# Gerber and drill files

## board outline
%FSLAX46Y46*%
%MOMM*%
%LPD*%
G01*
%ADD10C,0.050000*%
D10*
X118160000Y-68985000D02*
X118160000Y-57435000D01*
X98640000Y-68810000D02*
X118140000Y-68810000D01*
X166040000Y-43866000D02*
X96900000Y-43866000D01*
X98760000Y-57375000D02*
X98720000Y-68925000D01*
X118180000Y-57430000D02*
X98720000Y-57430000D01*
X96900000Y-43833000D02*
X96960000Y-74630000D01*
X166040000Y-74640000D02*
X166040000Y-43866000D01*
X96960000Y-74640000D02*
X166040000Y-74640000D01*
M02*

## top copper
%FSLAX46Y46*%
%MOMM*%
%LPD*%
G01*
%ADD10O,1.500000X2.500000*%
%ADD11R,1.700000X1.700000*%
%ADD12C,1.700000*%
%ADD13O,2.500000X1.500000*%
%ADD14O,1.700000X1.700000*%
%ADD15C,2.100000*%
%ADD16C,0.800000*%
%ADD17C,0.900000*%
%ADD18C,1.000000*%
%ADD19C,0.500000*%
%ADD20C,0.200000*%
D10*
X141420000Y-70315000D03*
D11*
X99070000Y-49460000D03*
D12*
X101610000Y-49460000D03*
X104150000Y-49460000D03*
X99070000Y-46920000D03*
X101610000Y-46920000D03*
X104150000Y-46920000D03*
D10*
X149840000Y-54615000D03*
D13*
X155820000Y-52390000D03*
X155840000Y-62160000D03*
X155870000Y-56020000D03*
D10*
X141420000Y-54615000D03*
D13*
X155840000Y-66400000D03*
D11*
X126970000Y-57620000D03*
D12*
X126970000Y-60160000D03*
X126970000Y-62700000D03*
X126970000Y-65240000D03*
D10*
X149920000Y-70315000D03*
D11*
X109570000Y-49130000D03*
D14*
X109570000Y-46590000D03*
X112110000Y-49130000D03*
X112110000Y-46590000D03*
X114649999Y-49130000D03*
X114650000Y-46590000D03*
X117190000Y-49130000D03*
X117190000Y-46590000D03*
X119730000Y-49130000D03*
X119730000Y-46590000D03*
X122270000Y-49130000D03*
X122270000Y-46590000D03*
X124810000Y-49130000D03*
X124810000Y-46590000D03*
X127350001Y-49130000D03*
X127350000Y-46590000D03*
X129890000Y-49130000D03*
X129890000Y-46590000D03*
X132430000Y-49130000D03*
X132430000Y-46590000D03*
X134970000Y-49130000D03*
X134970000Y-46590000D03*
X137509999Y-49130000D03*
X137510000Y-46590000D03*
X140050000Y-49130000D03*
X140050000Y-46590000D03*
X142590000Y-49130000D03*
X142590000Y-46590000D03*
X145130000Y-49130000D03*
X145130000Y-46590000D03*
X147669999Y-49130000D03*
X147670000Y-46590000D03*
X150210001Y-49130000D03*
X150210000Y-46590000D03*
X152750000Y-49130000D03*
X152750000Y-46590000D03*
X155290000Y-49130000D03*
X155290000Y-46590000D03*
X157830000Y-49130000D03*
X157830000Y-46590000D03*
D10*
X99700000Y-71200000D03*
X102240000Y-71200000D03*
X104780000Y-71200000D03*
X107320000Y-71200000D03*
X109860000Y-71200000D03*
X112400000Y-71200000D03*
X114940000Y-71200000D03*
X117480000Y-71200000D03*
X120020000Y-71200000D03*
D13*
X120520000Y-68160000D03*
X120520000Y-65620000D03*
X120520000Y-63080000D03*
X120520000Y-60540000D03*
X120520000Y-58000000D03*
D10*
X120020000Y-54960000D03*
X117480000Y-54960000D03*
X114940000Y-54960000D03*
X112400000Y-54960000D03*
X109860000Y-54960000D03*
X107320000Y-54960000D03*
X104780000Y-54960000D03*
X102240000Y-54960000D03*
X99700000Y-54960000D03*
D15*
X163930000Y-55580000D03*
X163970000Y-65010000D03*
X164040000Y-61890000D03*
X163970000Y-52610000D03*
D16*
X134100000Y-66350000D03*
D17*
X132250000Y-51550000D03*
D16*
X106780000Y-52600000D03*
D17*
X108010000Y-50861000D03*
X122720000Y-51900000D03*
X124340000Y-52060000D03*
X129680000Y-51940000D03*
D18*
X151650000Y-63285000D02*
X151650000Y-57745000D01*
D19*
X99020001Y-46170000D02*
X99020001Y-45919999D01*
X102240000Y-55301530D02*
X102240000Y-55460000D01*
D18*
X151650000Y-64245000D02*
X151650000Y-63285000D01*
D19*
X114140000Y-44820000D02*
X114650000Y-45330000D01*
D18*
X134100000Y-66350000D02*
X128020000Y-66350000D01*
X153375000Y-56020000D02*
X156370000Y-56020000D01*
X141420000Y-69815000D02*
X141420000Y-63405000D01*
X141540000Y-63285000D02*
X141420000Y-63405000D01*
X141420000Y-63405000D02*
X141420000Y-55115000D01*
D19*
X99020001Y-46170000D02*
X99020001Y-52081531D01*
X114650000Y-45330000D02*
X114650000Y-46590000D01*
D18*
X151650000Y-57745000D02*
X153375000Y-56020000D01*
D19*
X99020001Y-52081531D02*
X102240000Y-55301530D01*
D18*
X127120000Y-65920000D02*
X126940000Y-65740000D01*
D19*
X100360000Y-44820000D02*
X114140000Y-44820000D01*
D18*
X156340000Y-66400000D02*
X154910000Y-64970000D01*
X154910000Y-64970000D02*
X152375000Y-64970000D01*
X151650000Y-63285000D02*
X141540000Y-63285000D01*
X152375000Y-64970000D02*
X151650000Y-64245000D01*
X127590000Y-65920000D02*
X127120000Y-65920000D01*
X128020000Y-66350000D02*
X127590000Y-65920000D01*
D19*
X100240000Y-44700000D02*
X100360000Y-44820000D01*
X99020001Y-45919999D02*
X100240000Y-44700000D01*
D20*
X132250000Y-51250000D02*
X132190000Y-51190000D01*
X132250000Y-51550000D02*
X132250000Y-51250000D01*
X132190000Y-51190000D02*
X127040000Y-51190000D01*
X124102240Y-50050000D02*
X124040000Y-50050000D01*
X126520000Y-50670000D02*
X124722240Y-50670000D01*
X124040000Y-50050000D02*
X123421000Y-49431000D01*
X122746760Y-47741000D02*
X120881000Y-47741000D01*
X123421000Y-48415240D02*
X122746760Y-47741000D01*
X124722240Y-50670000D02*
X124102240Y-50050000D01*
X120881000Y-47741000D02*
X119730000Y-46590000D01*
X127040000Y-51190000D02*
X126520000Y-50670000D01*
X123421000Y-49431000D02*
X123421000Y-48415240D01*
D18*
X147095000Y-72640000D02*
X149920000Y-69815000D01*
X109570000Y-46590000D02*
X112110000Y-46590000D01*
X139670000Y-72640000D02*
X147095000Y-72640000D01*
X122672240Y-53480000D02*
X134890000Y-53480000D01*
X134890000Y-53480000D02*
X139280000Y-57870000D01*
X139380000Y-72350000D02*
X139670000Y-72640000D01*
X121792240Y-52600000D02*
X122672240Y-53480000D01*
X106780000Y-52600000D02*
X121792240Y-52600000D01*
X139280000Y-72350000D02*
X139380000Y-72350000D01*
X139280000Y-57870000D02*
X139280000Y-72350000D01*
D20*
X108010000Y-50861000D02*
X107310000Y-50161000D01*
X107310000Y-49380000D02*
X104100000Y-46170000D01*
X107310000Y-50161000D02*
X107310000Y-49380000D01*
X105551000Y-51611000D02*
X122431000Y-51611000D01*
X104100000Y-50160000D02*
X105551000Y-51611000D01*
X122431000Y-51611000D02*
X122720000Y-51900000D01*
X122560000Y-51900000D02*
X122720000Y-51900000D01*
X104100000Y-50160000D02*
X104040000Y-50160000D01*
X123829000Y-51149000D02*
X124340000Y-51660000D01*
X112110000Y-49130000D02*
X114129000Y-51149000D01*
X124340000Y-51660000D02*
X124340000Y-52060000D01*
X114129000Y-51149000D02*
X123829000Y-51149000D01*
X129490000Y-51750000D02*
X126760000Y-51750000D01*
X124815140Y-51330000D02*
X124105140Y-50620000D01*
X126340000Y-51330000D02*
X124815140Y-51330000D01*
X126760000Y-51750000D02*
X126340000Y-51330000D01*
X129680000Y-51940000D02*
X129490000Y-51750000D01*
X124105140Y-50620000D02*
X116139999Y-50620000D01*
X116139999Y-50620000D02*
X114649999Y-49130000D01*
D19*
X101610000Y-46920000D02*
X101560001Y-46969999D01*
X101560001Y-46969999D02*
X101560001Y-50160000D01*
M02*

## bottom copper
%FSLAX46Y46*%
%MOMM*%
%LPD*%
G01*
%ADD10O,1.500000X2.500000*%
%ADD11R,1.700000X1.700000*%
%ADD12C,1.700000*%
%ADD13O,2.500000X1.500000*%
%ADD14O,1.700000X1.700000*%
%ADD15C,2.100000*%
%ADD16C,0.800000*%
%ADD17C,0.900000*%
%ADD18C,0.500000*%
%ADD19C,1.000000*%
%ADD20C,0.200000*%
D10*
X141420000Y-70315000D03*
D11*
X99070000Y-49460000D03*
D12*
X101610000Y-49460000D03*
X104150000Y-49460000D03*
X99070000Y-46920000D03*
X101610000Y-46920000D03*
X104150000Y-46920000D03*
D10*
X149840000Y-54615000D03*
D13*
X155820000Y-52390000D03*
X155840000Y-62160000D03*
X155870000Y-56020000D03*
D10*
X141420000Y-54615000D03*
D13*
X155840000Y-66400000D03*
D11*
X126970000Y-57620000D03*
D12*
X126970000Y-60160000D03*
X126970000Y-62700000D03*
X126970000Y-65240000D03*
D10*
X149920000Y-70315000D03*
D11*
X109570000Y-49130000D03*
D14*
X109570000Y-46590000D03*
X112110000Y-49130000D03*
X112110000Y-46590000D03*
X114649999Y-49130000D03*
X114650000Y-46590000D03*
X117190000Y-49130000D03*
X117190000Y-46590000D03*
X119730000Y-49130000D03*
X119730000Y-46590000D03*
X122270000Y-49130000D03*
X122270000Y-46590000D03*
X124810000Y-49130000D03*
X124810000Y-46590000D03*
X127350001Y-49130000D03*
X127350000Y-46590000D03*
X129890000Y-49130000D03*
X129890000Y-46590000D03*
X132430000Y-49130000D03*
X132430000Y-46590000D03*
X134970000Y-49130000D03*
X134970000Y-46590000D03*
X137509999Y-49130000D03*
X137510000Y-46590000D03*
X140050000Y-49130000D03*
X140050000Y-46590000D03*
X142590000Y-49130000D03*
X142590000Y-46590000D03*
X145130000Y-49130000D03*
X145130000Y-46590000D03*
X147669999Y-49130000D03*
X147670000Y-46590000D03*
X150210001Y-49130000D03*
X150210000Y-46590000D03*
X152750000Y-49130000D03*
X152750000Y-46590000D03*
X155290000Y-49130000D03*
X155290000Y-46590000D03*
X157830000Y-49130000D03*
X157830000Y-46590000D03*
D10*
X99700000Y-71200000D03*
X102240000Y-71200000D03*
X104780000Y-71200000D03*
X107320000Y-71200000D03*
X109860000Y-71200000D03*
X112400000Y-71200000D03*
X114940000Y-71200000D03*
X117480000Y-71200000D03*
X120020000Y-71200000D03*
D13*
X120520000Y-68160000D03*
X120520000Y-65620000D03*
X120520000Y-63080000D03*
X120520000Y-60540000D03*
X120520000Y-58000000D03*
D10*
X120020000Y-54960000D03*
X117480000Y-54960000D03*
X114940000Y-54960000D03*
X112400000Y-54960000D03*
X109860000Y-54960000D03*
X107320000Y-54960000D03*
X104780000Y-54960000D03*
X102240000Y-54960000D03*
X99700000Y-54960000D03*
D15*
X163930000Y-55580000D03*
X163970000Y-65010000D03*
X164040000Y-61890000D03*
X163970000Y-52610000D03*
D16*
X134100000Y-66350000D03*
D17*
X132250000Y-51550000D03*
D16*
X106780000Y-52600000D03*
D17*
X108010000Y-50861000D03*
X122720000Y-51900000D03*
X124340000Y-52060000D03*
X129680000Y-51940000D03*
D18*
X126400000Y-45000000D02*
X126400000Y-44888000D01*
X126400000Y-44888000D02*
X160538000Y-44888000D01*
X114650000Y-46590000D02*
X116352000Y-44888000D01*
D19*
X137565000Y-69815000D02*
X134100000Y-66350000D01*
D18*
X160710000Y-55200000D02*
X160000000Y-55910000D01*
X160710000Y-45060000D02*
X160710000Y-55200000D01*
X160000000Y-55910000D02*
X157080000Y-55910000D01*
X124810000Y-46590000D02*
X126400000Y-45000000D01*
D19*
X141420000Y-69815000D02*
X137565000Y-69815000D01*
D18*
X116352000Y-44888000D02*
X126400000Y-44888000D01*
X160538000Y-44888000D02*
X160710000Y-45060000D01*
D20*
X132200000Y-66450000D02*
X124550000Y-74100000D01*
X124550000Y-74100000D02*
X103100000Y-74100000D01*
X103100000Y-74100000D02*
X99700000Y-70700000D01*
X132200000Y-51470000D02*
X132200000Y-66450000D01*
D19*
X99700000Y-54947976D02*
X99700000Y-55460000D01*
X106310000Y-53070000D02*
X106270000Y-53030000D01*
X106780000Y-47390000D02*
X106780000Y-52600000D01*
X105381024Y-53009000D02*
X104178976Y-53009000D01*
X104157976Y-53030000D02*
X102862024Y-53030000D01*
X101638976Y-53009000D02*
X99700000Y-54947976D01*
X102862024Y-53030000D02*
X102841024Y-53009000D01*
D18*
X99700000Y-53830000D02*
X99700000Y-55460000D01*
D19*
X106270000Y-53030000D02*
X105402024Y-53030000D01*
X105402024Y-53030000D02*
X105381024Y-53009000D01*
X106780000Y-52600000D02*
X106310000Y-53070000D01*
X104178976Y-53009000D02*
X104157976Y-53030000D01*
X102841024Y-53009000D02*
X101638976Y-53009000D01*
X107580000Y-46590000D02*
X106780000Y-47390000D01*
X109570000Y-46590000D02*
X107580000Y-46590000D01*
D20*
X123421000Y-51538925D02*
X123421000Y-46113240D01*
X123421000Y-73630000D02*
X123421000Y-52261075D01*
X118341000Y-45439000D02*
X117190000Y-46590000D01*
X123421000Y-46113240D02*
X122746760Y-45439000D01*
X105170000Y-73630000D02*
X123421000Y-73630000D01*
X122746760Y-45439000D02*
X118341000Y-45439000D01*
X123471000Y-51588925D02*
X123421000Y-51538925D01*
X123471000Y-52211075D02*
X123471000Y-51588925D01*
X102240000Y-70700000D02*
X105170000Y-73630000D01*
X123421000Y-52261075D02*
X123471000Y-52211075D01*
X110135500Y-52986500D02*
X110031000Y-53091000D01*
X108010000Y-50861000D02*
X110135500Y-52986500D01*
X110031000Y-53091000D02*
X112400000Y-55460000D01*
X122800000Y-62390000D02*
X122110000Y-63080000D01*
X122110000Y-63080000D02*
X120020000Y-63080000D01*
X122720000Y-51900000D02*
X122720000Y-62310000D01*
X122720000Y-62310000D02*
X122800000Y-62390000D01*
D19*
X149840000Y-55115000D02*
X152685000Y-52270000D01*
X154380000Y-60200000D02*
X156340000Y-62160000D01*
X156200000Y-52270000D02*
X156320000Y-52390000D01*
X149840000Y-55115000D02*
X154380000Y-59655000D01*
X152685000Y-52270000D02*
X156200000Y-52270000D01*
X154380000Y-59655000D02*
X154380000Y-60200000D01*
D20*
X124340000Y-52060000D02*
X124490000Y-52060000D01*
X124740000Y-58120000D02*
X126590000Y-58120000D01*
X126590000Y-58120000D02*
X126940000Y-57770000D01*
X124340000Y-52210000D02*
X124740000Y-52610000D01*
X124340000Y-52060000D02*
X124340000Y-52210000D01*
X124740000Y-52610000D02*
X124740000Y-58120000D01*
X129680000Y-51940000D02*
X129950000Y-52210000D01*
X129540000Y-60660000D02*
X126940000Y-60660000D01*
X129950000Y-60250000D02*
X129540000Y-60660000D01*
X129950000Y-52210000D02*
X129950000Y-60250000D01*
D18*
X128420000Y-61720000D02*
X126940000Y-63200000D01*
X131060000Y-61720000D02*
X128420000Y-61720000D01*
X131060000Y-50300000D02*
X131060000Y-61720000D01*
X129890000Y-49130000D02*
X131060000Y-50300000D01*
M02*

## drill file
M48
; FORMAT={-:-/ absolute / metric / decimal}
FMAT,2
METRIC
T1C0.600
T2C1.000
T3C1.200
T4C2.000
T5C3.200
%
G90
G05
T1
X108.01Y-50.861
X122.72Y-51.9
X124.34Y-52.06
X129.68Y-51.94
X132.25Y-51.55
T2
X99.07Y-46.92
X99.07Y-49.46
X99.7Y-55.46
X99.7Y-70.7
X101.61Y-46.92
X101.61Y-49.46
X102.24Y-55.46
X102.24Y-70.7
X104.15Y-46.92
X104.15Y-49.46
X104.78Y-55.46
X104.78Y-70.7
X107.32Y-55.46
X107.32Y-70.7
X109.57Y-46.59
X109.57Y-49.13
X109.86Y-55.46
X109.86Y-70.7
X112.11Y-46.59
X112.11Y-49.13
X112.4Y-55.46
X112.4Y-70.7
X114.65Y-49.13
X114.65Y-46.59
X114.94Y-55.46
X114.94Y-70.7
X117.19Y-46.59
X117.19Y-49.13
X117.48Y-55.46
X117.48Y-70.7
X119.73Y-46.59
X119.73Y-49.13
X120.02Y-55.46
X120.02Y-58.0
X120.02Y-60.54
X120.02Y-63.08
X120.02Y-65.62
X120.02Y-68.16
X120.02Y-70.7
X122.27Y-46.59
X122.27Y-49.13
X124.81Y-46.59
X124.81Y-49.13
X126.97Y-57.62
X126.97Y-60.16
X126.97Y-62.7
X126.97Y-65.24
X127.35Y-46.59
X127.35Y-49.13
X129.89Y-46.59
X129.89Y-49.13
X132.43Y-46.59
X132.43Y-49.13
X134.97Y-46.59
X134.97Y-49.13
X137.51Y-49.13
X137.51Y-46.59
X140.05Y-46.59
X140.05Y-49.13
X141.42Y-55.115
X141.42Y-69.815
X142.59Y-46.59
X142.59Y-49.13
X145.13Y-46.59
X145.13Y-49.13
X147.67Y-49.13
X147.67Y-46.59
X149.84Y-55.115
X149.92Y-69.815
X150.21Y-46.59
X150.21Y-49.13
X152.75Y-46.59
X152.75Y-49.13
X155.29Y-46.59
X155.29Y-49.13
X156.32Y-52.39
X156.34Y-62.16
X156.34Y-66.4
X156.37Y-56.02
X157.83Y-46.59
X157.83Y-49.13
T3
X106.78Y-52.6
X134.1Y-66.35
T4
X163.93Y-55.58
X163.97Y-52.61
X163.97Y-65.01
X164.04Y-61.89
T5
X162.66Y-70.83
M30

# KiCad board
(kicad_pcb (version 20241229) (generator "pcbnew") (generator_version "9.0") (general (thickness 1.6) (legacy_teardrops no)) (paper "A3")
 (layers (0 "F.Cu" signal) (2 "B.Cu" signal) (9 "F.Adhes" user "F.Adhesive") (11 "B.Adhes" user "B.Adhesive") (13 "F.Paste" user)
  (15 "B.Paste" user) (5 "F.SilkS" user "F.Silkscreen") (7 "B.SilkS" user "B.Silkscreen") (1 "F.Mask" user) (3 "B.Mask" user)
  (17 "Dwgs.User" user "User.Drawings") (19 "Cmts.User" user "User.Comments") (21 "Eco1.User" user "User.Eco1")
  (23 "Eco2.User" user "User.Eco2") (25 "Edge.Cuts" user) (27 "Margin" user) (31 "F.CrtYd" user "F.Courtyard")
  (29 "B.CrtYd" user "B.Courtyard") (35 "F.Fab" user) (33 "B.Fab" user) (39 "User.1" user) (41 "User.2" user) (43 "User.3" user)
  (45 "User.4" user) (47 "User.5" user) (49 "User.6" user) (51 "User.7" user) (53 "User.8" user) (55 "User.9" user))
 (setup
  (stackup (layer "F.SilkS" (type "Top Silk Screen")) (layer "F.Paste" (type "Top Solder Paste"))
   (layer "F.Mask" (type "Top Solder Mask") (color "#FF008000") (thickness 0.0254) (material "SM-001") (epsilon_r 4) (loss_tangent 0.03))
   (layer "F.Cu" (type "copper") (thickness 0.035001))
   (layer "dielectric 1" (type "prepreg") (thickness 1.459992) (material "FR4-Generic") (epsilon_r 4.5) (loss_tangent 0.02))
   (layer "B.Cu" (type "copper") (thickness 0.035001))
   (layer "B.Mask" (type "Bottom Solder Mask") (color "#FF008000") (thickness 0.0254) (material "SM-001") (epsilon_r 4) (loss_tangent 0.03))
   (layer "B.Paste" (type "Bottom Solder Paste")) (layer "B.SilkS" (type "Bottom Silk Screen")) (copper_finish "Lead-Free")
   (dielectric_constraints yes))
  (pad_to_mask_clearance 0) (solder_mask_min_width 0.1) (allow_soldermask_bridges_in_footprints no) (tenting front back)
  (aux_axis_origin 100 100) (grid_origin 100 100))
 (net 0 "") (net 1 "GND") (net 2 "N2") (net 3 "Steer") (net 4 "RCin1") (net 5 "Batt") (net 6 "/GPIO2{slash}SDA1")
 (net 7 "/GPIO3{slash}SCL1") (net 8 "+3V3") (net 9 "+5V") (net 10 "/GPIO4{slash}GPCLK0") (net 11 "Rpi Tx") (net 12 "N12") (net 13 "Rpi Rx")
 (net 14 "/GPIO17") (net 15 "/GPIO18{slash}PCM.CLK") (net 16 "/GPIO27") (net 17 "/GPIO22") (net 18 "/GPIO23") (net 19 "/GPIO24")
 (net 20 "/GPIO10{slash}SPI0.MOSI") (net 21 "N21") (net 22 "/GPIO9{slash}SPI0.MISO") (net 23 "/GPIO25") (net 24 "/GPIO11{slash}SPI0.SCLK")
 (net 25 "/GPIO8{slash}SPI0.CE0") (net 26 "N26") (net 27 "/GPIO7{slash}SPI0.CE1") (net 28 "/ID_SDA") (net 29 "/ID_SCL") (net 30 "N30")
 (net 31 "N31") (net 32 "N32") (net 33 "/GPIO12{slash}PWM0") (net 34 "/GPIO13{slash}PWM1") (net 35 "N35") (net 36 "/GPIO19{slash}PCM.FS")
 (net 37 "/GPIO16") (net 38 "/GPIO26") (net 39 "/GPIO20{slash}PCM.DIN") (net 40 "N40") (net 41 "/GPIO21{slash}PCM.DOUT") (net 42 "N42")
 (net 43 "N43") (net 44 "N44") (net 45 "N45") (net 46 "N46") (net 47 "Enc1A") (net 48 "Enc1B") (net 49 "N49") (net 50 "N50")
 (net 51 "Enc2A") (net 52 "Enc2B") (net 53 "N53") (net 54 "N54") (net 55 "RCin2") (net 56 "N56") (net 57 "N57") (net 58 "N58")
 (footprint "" (layer "F.Cu") (at 141.42 69.815 180)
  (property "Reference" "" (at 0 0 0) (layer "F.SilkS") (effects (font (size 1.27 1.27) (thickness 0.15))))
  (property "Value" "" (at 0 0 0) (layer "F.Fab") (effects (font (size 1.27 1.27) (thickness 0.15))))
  (pad "15" thru_hole oval (at 0 0 90) (size 2.5 1.5) (drill 1 (offset -0.5 0)) (layers "*.Cu" "*.Mask") (remove_unused_layers no)
   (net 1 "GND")))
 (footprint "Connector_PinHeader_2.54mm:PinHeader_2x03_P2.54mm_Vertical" (layer "F.Cu") (at 99.07 49.46 90)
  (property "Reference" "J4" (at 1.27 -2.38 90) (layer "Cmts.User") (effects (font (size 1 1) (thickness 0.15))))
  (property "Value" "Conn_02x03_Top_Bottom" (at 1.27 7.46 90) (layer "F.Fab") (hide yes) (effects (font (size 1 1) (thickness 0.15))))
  (pad "1" thru_hole rect (at 0 0 90) (size 1.7 1.7) (drill 1) (layers "*.Cu" "*.Mask") (remove_unused_layers no) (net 1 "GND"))
  (pad "2" thru_hole circle (at 0 2.54 90) (size 1.7 1.7) (drill 1) (layers "*.Cu" "*.Mask") (remove_unused_layers no) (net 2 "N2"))
  (pad "3" thru_hole circle (at 0 5.08 90) (size 1.7 1.7) (drill 1) (layers "*.Cu" "*.Mask") (remove_unused_layers no) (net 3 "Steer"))
  (pad "4" thru_hole circle (at 2.54 0 90) (size 1.7 1.7) (drill 1) (layers "*.Cu" "*.Mask") (remove_unused_layers no) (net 1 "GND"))
  (pad "5" thru_hole circle (at 2.54 2.54 90) (size 1.7 1.7) (drill 1) (layers "*.Cu" "*.Mask") (remove_unused_layers no) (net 2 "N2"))
  (pad "6" thru_hole circle (at 2.54 5.08 90) (size 1.7 1.7) (drill 1) (layers "*.Cu" "*.Mask") (remove_unused_layers no) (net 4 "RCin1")))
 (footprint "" (layer "F.Cu") (at 149.84 55.115)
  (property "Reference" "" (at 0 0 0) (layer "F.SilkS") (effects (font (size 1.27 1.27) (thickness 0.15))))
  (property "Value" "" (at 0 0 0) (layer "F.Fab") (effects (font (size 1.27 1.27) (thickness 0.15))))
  (pad "15" thru_hole oval (at 0 0 270) (size 2.5 1.5) (drill 1 (offset -0.5 0)) (layers "*.Cu" "*.Mask") (remove_unused_layers no)
   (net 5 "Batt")))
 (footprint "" (layer "F.Cu") (at 156.32 52.39 90)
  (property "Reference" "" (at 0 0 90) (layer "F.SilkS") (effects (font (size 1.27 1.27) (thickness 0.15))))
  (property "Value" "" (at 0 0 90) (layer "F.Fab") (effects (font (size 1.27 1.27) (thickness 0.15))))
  (pad "15" thru_hole oval (at 0 0) (size 2.5 1.5) (drill 1 (offset -0.5 0)) (layers "*.Cu" "*.Mask") (remove_unused_layers no)
   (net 5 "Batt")))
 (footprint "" (layer "F.Cu") (at 156.34 62.16)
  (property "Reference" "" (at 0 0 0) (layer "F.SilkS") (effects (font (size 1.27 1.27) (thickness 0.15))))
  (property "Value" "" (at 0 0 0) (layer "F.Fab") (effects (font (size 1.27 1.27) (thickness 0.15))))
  (pad "15" thru_hole oval (at 0 0) (size 2.5 1.5) (drill 1 (offset -0.5 0)) (layers "*.Cu" "*.Mask") (remove_unused_layers no)
   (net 5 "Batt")))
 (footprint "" (layer "F.Cu") (at 156.37 56.02 -90)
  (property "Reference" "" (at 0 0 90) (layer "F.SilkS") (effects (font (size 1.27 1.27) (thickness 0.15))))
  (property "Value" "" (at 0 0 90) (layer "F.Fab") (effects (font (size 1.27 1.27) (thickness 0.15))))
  (pad "15" thru_hole oval (at 0 0) (size 2.5 1.5) (drill 1 (offset -0.5 0)) (layers "*.Cu" "*.Mask") (remove_unused_layers no)
   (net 1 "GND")))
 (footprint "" (layer "F.Cu") (at 141.42 55.115)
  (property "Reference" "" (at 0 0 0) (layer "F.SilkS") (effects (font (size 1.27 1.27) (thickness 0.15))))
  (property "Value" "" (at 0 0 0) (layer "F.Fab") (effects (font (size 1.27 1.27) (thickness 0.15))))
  (pad "15" thru_hole oval (at 0 0 270) (size 2.5 1.5) (drill 1 (offset -0.5 0)) (layers "*.Cu" "*.Mask") (remove_unused_layers no)
   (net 1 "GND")))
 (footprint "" (layer "F.Cu") (at 156.34 66.4)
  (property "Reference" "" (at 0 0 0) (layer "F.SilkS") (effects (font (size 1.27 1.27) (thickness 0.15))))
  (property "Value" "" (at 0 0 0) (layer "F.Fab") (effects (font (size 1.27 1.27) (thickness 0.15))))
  (pad "15" thru_hole oval (at 0 0) (size 2.5 1.5) (drill 1 (offset -0.5 0)) (layers "*.Cu" "*.Mask") (remove_unused_layers no)
   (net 1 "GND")))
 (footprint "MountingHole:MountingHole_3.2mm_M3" (layer "F.Cu") (at 162.66 70.83)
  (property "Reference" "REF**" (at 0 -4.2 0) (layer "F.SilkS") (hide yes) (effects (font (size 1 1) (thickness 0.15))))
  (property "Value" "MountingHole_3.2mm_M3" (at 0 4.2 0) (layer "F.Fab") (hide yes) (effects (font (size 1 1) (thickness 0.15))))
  (pad "" np_thru_hole circle (at 0 0) (size 3.2 3.2) (drill 3.2) (layers "*.Cu" "*.Mask")))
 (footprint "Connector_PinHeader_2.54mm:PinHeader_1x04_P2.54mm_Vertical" (layer "F.Cu") (at 126.97 57.62)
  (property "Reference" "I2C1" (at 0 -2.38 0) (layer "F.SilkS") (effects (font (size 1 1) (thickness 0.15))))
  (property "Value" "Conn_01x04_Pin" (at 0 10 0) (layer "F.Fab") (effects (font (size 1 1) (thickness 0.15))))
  (pad "1" thru_hole rect (at 0 0) (size 1.7 1.7) (drill 1) (layers "*.Cu" "*.Mask") (remove_unused_layers no) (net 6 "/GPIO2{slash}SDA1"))
  (pad "2" thru_hole circle (at 0 2.54) (size 1.7 1.7) (drill 1) (layers "*.Cu" "*.Mask") (remove_unused_layers no)
   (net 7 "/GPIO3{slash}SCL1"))
  (pad "3" thru_hole circle (at 0 5.08) (size 1.7 1.7) (drill 1) (layers "*.Cu" "*.Mask") (remove_unused_layers no) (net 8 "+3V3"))
  (pad "4" thru_hole circle (at 0 7.62) (size 1.7 1.7) (drill 1) (layers "*.Cu" "*.Mask") (remove_unused_layers no) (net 1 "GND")))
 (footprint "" (layer "F.Cu") (at 149.92 69.815 180)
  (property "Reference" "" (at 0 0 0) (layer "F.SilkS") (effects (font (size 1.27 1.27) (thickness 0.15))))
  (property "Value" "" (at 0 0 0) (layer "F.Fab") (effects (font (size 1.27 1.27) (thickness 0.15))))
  (pad "15" thru_hole oval (at 0 0 90) (size 2.5 1.5) (drill 1 (offset -0.5 0)) (layers "*.Cu" "*.Mask") (remove_unused_layers no)
   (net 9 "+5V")))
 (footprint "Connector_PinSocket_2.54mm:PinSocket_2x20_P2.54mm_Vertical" (layer "B.Cu") (at 109.57 49.13 -90)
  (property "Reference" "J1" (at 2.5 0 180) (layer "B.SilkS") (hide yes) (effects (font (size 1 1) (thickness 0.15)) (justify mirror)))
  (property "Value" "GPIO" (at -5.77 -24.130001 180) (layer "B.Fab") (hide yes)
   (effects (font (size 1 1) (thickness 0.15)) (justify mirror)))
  (pad "1" thru_hole rect (at 0 0 270) (size 1.7 1.7) (drill 1) (layers "*.Cu" "*.Mask") (remove_unused_layers no) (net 8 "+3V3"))
  (pad "2" thru_hole oval (at -2.54 0 270) (size 1.7 1.7) (drill 1) (layers "*.Cu" "*.Mask") (remove_unused_layers no) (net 9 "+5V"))
  (pad "3" thru_hole oval (at 0 -2.54 270) (size 1.7 1.7) (drill 1) (layers "*.Cu" "*.Mask") (remove_unused_layers no)
   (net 6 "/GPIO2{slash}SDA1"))
  (pad "4" thru_hole oval (at -2.54 -2.54 270) (size 1.7 1.7) (drill 1) (layers "*.Cu" "*.Mask") (remove_unused_layers no) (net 9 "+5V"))
  (pad "5" thru_hole oval (at 0 -5.079999 270) (size 1.7 1.7) (drill 1) (layers "*.Cu" "*.Mask") (remove_unused_layers no)
   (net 7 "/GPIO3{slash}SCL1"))
  (pad "6" thru_hole oval (at -2.54 -5.08 270) (size 1.7 1.7) (drill 1) (layers "*.Cu" "*.Mask") (remove_unused_layers no) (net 1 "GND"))
  (pad "7" thru_hole oval (at 0 -7.62 270) (size 1.7 1.7) (drill 1) (layers "*.Cu" "*.Mask") (remove_unused_layers no)
   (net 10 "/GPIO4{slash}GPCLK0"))
  (pad "8" thru_hole oval (at -2.54 -7.62 270) (size 1.7 1.7) (drill 1) (layers "*.Cu" "*.Mask") (remove_unused_layers no) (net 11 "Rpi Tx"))
  (pad "9" thru_hole oval (at 0 -10.16 270) (size 1.7 1.7) (drill 1) (layers "*.Cu" "*.Mask") (remove_unused_layers no) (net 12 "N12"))
  (pad "10" thru_hole oval (at -2.54 -10.16 270) (size 1.7 1.7) (drill 1) (layers "*.Cu" "*.Mask") (remove_unused_layers no)
   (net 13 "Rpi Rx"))
  (pad "11" thru_hole oval (at 0 -12.7 270) (size 1.7 1.7) (drill 1) (layers "*.Cu" "*.Mask") (remove_unused_layers no) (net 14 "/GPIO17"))
  (pad "12" thru_hole oval (at -2.54 -12.7 270) (size 1.7 1.7) (drill 1) (layers "*.Cu" "*.Mask") (remove_unused_layers no)
   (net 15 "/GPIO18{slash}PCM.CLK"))
  (pad "13" thru_hole oval (at 0 -15.24 270) (size 1.7 1.7) (drill 1) (layers "*.Cu" "*.Mask") (remove_unused_layers no) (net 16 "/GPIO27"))
  (pad "14" thru_hole oval (at -2.54 -15.24 270) (size 1.7 1.7) (drill 1) (layers "*.Cu" "*.Mask") (remove_unused_layers no) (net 1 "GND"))
  (pad "15" thru_hole oval (at 0 -17.780001 270) (size 1.7 1.7) (drill 1) (layers "*.Cu" "*.Mask") (remove_unused_layers no)
   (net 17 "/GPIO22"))
  (pad "16" thru_hole oval (at -2.54 -17.78 270) (size 1.7 1.7) (drill 1) (layers "*.Cu" "*.Mask") (remove_unused_layers no)
   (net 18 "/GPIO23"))
  (pad "17" thru_hole oval (at 0 -20.32 270) (size 1.7 1.7) (drill 1) (layers "*.Cu" "*.Mask") (remove_unused_layers no) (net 8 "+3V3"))
  (pad "18" thru_hole oval (at -2.54 -20.32 270) (size 1.7 1.7) (drill 1) (layers "*.Cu" "*.Mask") (remove_unused_layers no)
   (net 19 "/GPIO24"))
  (pad "19" thru_hole oval (at 0 -22.86 270) (size 1.7 1.7) (drill 1) (layers "*.Cu" "*.Mask") (remove_unused_layers no)
   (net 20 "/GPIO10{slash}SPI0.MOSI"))
  (pad "20" thru_hole oval (at -2.54 -22.86 270) (size 1.7 1.7) (drill 1) (layers "*.Cu" "*.Mask") (remove_unused_layers no) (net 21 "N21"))
  (pad "21" thru_hole oval (at 0 -25.4 270) (size 1.7 1.7) (drill 1) (layers "*.Cu" "*.Mask") (remove_unused_layers no)
   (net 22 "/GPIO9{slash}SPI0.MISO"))
  (pad "22" thru_hole oval (at -2.54 -25.4 270) (size 1.7 1.7) (drill 1) (layers "*.Cu" "*.Mask") (remove_unused_layers no)
   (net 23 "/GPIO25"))
  (pad "23" thru_hole oval (at 0 -27.939999 270) (size 1.7 1.7) (drill 1) (layers "*.Cu" "*.Mask") (remove_unused_layers no)
   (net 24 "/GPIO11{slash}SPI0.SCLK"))
  (pad "24" thru_hole oval (at -2.54 -27.94 270) (size 1.7 1.7) (drill 1) (layers "*.Cu" "*.Mask") (remove_unused_layers no)
   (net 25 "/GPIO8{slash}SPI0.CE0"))
  (pad "25" thru_hole oval (at 0 -30.48 270) (size 1.7 1.7) (drill 1) (layers "*.Cu" "*.Mask") (remove_unused_layers no) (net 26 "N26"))
  (pad "26" thru_hole oval (at -2.54 -30.48 270) (size 1.7 1.7) (drill 1) (layers "*.Cu" "*.Mask") (remove_unused_layers no)
   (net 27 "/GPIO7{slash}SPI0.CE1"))
  (pad "27" thru_hole oval (at 0 -33.02 270) (size 1.7 1.7) (drill 1) (layers "*.Cu" "*.Mask") (remove_unused_layers no) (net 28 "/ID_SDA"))
  (pad "28" thru_hole oval (at -2.54 -33.02 270) (size 1.7 1.7) (drill 1) (layers "*.Cu" "*.Mask") (remove_unused_layers no)
   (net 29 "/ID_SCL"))
  (pad "29" thru_hole oval (at 0 -35.56 270) (size 1.7 1.7) (drill 1) (layers "*.Cu" "*.Mask") (remove_unused_layers no) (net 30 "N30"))
  (pad "30" thru_hole oval (at -2.54 -35.56 270) (size 1.7 1.7) (drill 1) (layers "*.Cu" "*.Mask") (remove_unused_layers no) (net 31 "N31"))
  (pad "31" thru_hole oval (at 0 -38.099999 270) (size 1.7 1.7) (drill 1) (layers "*.Cu" "*.Mask") (remove_unused_layers no) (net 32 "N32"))
  (pad "32" thru_hole oval (at -2.54 -38.1 270) (size 1.7 1.7) (drill 1) (layers "*.Cu" "*.Mask") (remove_unused_layers no)
   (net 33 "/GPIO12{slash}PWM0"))
  (pad "33" thru_hole oval (at 0 -40.640001 270) (size 1.7 1.7) (drill 1) (layers "*.Cu" "*.Mask") (remove_unused_layers no)
   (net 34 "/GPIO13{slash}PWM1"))
  (pad "34" thru_hole oval (at -2.54 -40.64 270) (size 1.7 1.7) (drill 1) (layers "*.Cu" "*.Mask") (remove_unused_layers no) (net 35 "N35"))
  (pad "35" thru_hole oval (at 0 -43.18 270) (size 1.7 1.7) (drill 1) (layers "*.Cu" "*.Mask") (remove_unused_layers no)
   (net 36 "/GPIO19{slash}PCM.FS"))
  (pad "36" thru_hole oval (at -2.54 -43.18 270) (size 1.7 1.7) (drill 1) (layers "*.Cu" "*.Mask") (remove_unused_layers no)
   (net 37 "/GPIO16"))
  (pad "37" thru_hole oval (at 0 -45.72 270) (size 1.7 1.7) (drill 1) (layers "*.Cu" "*.Mask") (remove_unused_layers no) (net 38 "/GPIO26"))
  (pad "38" thru_hole oval (at -2.54 -45.72 270) (size 1.7 1.7) (drill 1) (layers "*.Cu" "*.Mask") (remove_unused_layers no)
   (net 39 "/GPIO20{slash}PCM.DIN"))
  (pad "39" thru_hole oval (at 0 -48.26 270) (size 1.7 1.7) (drill 1) (layers "*.Cu" "*.Mask") (remove_unused_layers no) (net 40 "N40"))
  (pad "40" thru_hole oval (at -2.54 -48.26 270) (size 1.7 1.7) (drill 1) (layers "*.Cu" "*.Mask") (remove_unused_layers no)
   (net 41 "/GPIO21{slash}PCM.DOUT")))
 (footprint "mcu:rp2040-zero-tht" (layer "B.Cu") (at 109.86 63.08 -90)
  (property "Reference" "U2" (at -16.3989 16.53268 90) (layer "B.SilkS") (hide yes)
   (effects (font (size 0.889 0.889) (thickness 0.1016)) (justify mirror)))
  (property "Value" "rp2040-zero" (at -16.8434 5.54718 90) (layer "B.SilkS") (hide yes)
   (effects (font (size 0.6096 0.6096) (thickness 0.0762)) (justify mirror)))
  (pad "1" thru_hole oval (at 7.62 10.16 90) (size 2.5 1.5) (drill 1 (offset -0.5 0)) (layers "*.Cu" "*.Mask") (remove_unused_layers no)
   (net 13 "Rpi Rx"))
  (pad "2" thru_hole oval (at 7.62 7.62 90) (size 2.5 1.5) (drill 1 (offset -0.5 0)) (layers "*.Cu" "*.Mask") (remove_unused_layers no)
   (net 11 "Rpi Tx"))
  (pad "3" thru_hole oval (at 7.62 5.08 90) (size 2.5 1.5) (drill 1 (offset -0.5 0)) (layers "*.Cu" "*.Mask") (remove_unused_layers no)
   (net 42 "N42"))
  (pad "4" thru_hole oval (at 7.62 2.54 90) (size 2.5 1.5) (drill 1 (offset -0.5 0)) (layers "*.Cu" "*.Mask") (remove_unused_layers no)
   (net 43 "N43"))
  (pad "5" thru_hole oval (at 7.62 0 90) (size 2.5 1.5) (drill 1 (offset -0.5 0)) (layers "*.Cu" "*.Mask") (remove_unused_layers no)
   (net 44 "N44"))
  (pad "6" thru_hole oval (at 7.62 -2.54 90) (size 2.5 1.5) (drill 1 (offset -0.5 0)) (layers "*.Cu" "*.Mask") (remove_unused_layers no)
   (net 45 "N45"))
  (pad "7" thru_hole oval (at 7.62 -5.08 90) (size 2.5 1.5) (drill 1 (offset -0.5 0)) (layers "*.Cu" "*.Mask") (remove_unused_layers no)
   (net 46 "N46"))
  (pad "8" thru_hole oval (at 7.62 -7.62 90) (size 2.5 1.5) (drill 1 (offset -0.5 0)) (layers "*.Cu" "*.Mask") (remove_unused_layers no)
   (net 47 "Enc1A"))
  (pad "9" thru_hole oval (at 7.62 -10.16 90) (size 2.5 1.5) (drill 1 (offset -0.5 0)) (layers "*.Cu" "*.Mask") (remove_unused_layers no)
   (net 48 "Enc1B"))
  (pad "10" thru_hole oval (at 5.08 -10.16 180) (size 2.5 1.5) (drill 1 (offset -0.5 0)) (layers "*.Cu" "*.Mask") (remove_unused_layers no)
   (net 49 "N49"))
  (pad "11" thru_hole oval (at 2.54 -10.16 180) (size 2.5 1.5) (drill 1 (offset -0.5 0)) (layers "*.Cu" "*.Mask") (remove_unused_layers no)
   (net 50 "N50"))
  (pad "12" thru_hole oval (at 0 -10.16 180) (size 2.5 1.5) (drill 1 (offset -0.5 0)) (layers "*.Cu" "*.Mask") (remove_unused_layers no)
   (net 3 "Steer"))
  (pad "13" thru_hole oval (at -2.54 -10.16 180) (size 2.5 1.5) (drill 1 (offset -0.5 0)) (layers "*.Cu" "*.Mask") (remove_unused_layers no)
   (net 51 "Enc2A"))
  (pad "14" thru_hole oval (at -5.08 -10.16 180) (size 2.5 1.5) (drill 1 (offset -0.5 0)) (layers "*.Cu" "*.Mask") (remove_unused_layers no)
   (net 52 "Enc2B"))
  (pad "15" thru_hole oval (at -7.62 -10.16 270) (size 2.5 1.5) (drill 1 (offset -0.5 0)) (layers "*.Cu" "*.Mask") (remove_unused_layers no)
   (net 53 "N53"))
  (pad "16" thru_hole oval (at -7.62 -7.62 270) (size 2.5 1.5) (drill 1 (offset -0.5 0)) (layers "*.Cu" "*.Mask") (remove_unused_layers no)
   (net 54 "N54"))
  (pad "17" thru_hole oval (at -7.62 -5.08 270) (size 2.5 1.5) (drill 1 (offset -0.5 0)) (layers "*.Cu" "*.Mask") (remove_unused_layers no)
   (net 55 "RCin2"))
  (pad "18" thru_hole oval (at -7.62 -2.54 270) (size 2.5 1.5) (drill 1 (offset -0.5 0)) (layers "*.Cu" "*.Mask") (remove_unused_layers no)
   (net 4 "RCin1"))
  (pad "19" thru_hole oval (at -7.62 0 270) (size 2.5 1.5) (drill 1 (offset -0.5 0)) (layers "*.Cu" "*.Mask") (remove_unused_layers no)
   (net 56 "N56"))
  (pad "20" thru_hole oval (at -7.62 2.54 270) (size 2.5 1.5) (drill 1 (offset -0.5 0)) (layers "*.Cu" "*.Mask") (remove_unused_layers no)
   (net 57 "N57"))
  (pad "21" thru_hole oval (at -7.62 5.08 270) (size 2.5 1.5) (drill 1 (offset -0.5 0)) (layers "*.Cu" "*.Mask") (remove_unused_layers no)
   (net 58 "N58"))
  (pad "22" thru_hole oval (at -7.62 7.62 270) (size 2.5 1.5) (drill 1 (offset -0.5 0)) (layers "*.Cu" "*.Mask") (remove_unused_layers no)
   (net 1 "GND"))
  (pad "23" thru_hole oval (at -7.62 10.16 270) (size 2.5 1.5) (drill 1 (offset -0.5 0)) (layers "*.Cu" "*.Mask") (remove_unused_layers no)
   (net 9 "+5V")))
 (gr_line (start 118.16 68.985) (end 118.16 57.435) (stroke (width 0.05) (type default)) (layer "Edge.Cuts"))
 (gr_line (start 98.64 68.81) (end 118.14 68.81) (stroke (width 0.05) (type default)) (layer "Edge.Cuts"))
 (gr_line (start 166.04 43.866) (end 96.9 43.866) (stroke (width 0.05) (type default)) (layer "Edge.Cuts"))
 (gr_line (start 98.76 57.375) (end 98.72 68.925) (stroke (width 0.05) (type default)) (layer "Edge.Cuts"))
 (gr_line (start 118.18 57.43) (end 98.72 57.43) (stroke (width 0.05) (type default)) (layer "Edge.Cuts"))
 (gr_line (start 96.9 43.833) (end 96.96 74.63) (stroke (width 0.05) (type default)) (layer "Edge.Cuts"))
 (gr_line (start 166.04 74.64) (end 166.04 43.866) (stroke (width 0.05) (type default)) (layer "Edge.Cuts"))
 (gr_line (start 96.96 74.64) (end 166.04 74.64) (stroke (width 0.05) (type default)) (layer "Edge.Cuts"))
 (via (at 163.93 55.58) (size 2.1) (drill 2) (layers "F.Cu" "B.Cu") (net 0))
 (via (at 163.97 65.01) (size 2.1) (drill 2) (layers "F.Cu" "B.Cu") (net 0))
 (via (at 164.04 61.89) (size 2.1) (drill 2) (layers "F.Cu" "B.Cu") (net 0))
 (via (at 163.97 52.61) (size 2.1) (drill 2) (layers "F.Cu" "B.Cu") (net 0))
 (segment (start 151.65 63.285) (end 151.65 57.745) (width 1) (layer "F.Cu") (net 1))
 (segment (start 99.020001 46.17) (end 99.020001 45.919999) (width 0.5) (layer "F.Cu") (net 1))
 (segment (start 102.24 55.30153) (end 102.24 55.46) (width 0.5) (layer "F.Cu") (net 1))
 (segment (start 151.65 64.245) (end 151.65 63.285) (width 1) (layer "F.Cu") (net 1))
 (segment (start 114.14 44.82) (end 114.65 45.33) (width 0.5) (layer "F.Cu") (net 1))
 (segment (start 134.1 66.35) (end 128.02 66.35) (width 1) (layer "F.Cu") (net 1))
 (segment (start 153.375 56.02) (end 156.37 56.02) (width 1) (layer "F.Cu") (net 1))
 (segment (start 141.42 69.815) (end 141.42 63.405) (width 1) (layer "F.Cu") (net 1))
 (segment (start 141.54 63.285) (end 141.42 63.405) (width 1) (layer "F.Cu") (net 1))
 (segment (start 141.42 63.405) (end 141.42 55.115) (width 1) (layer "F.Cu") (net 1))
 (segment (start 99.020001 46.17) (end 99.020001 52.081531) (width 0.5) (layer "F.Cu") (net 1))
 (segment (start 114.65 45.33) (end 114.65 46.59) (width 0.5) (layer "F.Cu") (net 1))
 (segment (start 151.65 57.745) (end 153.375 56.02) (width 1) (layer "F.Cu") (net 1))
 (segment (start 99.020001 52.081531) (end 102.24 55.30153) (width 0.5) (layer "F.Cu") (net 1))
 (segment (start 127.12 65.92) (end 126.94 65.74) (width 1) (layer "F.Cu") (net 1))
 (segment (start 100.36 44.82) (end 114.14 44.82) (width 0.5) (layer "F.Cu") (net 1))
 (segment (start 156.34 66.4) (end 154.91 64.97) (width 1) (layer "F.Cu") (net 1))
 (segment (start 154.91 64.97) (end 152.375 64.97) (width 1) (layer "F.Cu") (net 1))
 (segment (start 151.65 63.285) (end 141.54 63.285) (width 1) (layer "F.Cu") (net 1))
 (segment (start 152.375 64.97) (end 151.65 64.245) (width 1) (layer "F.Cu") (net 1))
 (segment (start 127.59 65.92) (end 127.12 65.92) (width 1) (layer "F.Cu") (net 1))
 (segment (start 128.02 66.35) (end 127.59 65.92) (width 1) (layer "F.Cu") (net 1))
 (segment (start 100.24 44.7) (end 100.36 44.82) (width 0.5) (layer "F.Cu") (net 1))
 (segment (start 99.020001 45.919999) (end 100.24 44.7) (width 0.5) (layer "F.Cu") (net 1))
 (via (at 134.1 66.35) (size 0.8) (drill 1.2) (layers "F.Cu" "B.Cu") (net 1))
 (segment (start 126.4 45) (end 126.4 44.888) (width 0.5) (layer "B.Cu") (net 1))
 (segment (start 126.4 44.888) (end 160.538 44.888) (width 0.5) (layer "B.Cu") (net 1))
 (segment (start 114.65 46.59) (end 116.352 44.888) (width 0.5) (layer "B.Cu") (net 1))
 (segment (start 137.565 69.815) (end 134.1 66.35) (width 1) (layer "B.Cu") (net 1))
 (segment (start 160.71 55.2) (end 160 55.91) (width 0.5) (layer "B.Cu") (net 1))
 (segment (start 160.71 45.06) (end 160.71 55.2) (width 0.5) (layer "B.Cu") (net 1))
 (segment (start 160 55.91) (end 157.08 55.91) (width 0.5) (layer "B.Cu") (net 1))
 (segment (start 124.81 46.59) (end 126.4 45) (width 0.5) (layer "B.Cu") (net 1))
 (segment (start 141.42 69.815) (end 137.565 69.815) (width 1) (layer "B.Cu") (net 1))
 (segment (start 116.352 44.888) (end 126.4 44.888) (width 0.5) (layer "B.Cu") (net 1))
 (segment (start 160.538 44.888) (end 160.71 45.06) (width 0.5) (layer "B.Cu") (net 1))
 (segment (start 132.25 51.25) (end 132.19 51.19) (width 0.2) (layer "F.Cu") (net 13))
 (segment (start 132.25 51.55) (end 132.25 51.25) (width 0.2) (layer "F.Cu") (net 13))
 (segment (start 132.19 51.19) (end 127.04 51.19) (width 0.2) (layer "F.Cu") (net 13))
 (segment (start 124.10224 50.05) (end 124.04 50.05) (width 0.2) (layer "F.Cu") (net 13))
 (segment (start 126.52 50.67) (end 124.72224 50.67) (width 0.2) (layer "F.Cu") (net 13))
 (segment (start 124.04 50.05) (end 123.421 49.431) (width 0.2) (layer "F.Cu") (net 13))
 (segment (start 122.74676 47.741) (end 120.881 47.741) (width 0.2) (layer "F.Cu") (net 13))
 (segment (start 123.421 48.41524) (end 122.74676 47.741) (width 0.2) (layer "F.Cu") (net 13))
 (segment (start 124.72224 50.67) (end 124.10224 50.05) (width 0.2) (layer "F.Cu") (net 13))
 (segment (start 120.881 47.741) (end 119.73 46.59) (width 0.2) (layer "F.Cu") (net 13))
 (segment (start 127.04 51.19) (end 126.52 50.67) (width 0.2) (layer "F.Cu") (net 13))
 (segment (start 123.421 49.431) (end 123.421 48.41524) (width 0.2) (layer "F.Cu") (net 13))
 (via (at 132.25 51.55) (size 0.9) (drill 0.6) (layers "F.Cu" "B.Cu") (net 13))
 (segment (start 132.2 66.45) (end 124.55 74.1) (width 0.2) (layer "B.Cu") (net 13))
 (segment (start 124.55 74.1) (end 103.1 74.1) (width 0.2) (layer "B.Cu") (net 13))
 (segment (start 103.1 74.1) (end 99.7 70.7) (width 0.2) (layer "B.Cu") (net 13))
 (segment (start 132.2 51.47) (end 132.2 66.45) (width 0.2) (layer "B.Cu") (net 13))
 (segment (start 147.095 72.64) (end 149.92 69.815) (width 1) (layer "F.Cu") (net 9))
 (segment (start 109.57 46.59) (end 112.11 46.59) (width 1) (layer "F.Cu") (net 9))
 (segment (start 139.67 72.64) (end 147.095 72.64) (width 1) (layer "F.Cu") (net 9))
 (segment (start 122.67224 53.48) (end 134.89 53.48) (width 1) (layer "F.Cu") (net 9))
 (segment (start 134.89 53.48) (end 139.28 57.87) (width 1) (layer "F.Cu") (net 9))
 (segment (start 139.38 72.35) (end 139.67 72.64) (width 1) (layer "F.Cu") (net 9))
 (segment (start 121.79224 52.6) (end 122.67224 53.48) (width 1) (layer "F.Cu") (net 9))
 (segment (start 106.78 52.6) (end 121.79224 52.6) (width 1) (layer "F.Cu") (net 9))
 (segment (start 139.28 72.35) (end 139.38 72.35) (width 1) (layer "F.Cu") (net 9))
 (segment (start 139.28 57.87) (end 139.28 72.35) (width 1) (layer "F.Cu") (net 9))
 (via (at 106.78 52.6) (size 0.8) (drill 1.2) (layers "F.Cu" "B.Cu") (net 9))
 (segment (start 99.7 54.947976) (end 99.7 55.46) (width 1) (layer "B.Cu") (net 9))
 (segment (start 106.31 53.07) (end 106.27 53.03) (width 1) (layer "B.Cu") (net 9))
 (segment (start 106.78 47.39) (end 106.78 52.6) (width 1) (layer "B.Cu") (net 9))
 (segment (start 105.381024 53.009) (end 104.178976 53.009) (width 1) (layer "B.Cu") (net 9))
 (segment (start 104.157976 53.03) (end 102.862024 53.03) (width 1) (layer "B.Cu") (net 9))
 (segment (start 101.638976 53.009) (end 99.7 54.947976) (width 1) (layer "B.Cu") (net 9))
 (segment (start 102.862024 53.03) (end 102.841024 53.009) (width 1) (layer "B.Cu") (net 9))
 (segment (start 99.7 53.83) (end 99.7 55.46) (width 0.5) (layer "B.Cu") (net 9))
 (segment (start 106.27 53.03) (end 105.402024 53.03) (width 1) (layer "B.Cu") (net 9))
 (segment (start 105.402024 53.03) (end 105.381024 53.009) (width 1) (layer "B.Cu") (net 9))
 (segment (start 106.78 52.6) (end 106.31 53.07) (width 1) (layer "B.Cu") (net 9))
 (segment (start 104.178976 53.009) (end 104.157976 53.03) (width 1) (layer "B.Cu") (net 9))
 (segment (start 102.841024 53.009) (end 101.638976 53.009) (width 1) (layer "B.Cu") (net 9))
 (segment (start 107.58 46.59) (end 106.78 47.39) (width 1) (layer "B.Cu") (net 9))
 (segment (start 109.57 46.59) (end 107.58 46.59) (width 1) (layer "B.Cu") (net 9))
 (segment (start 123.421 51.538925) (end 123.421 46.11324) (width 0.2) (layer "B.Cu") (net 11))
 (segment (start 123.421 73.63) (end 123.421 52.261075) (width 0.2) (layer "B.Cu") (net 11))
 (segment (start 118.341 45.439) (end 117.19 46.59) (width 0.2) (layer "B.Cu") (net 11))
 (segment (start 123.421 46.11324) (end 122.74676 45.439) (width 0.2) (layer "B.Cu") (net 11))
 (segment (start 105.17 73.63) (end 123.421 73.63) (width 0.2) (layer "B.Cu") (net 11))
 (segment (start 122.74676 45.439) (end 118.341 45.439) (width 0.2) (layer "B.Cu") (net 11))
 (segment (start 123.471 51.588925) (end 123.421 51.538925) (width 0.2) (layer "B.Cu") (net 11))
 (segment (start 123.471 52.211075) (end 123.471 51.588925) (width 0.2) (layer "B.Cu") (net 11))
 (segment (start 102.24 70.7) (end 105.17 73.63) (width 0.2) (layer "B.Cu") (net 11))
 (segment (start 123.421 52.261075) (end 123.471 52.211075) (width 0.2) (layer "B.Cu") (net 11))
 (segment (start 108.01 50.861) (end 107.31 50.161) (width 0.2) (layer "F.Cu") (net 4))
 (segment (start 107.31 49.38) (end 104.1 46.17) (width 0.2) (layer "F.Cu") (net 4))
 (segment (start 107.31 50.161) (end 107.31 49.38) (width 0.2) (layer "F.Cu") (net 4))
 (via (at 108.01 50.861) (size 0.9) (drill 0.6) (layers "F.Cu" "B.Cu") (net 4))
 (segment (start 110.1355 52.9865) (end 110.031 53.091) (width 0.2) (layer "B.Cu") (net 4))
 (segment (start 108.01 50.861) (end 110.1355 52.9865) (width 0.2) (layer "B.Cu") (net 4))
 (segment (start 110.031 53.091) (end 112.4 55.46) (width 0.2) (layer "B.Cu") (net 4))
 (segment (start 105.551 51.611) (end 122.431 51.611) (width 0.2) (layer "F.Cu") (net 3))
 (segment (start 104.1 50.16) (end 105.551 51.611) (width 0.2) (layer "F.Cu") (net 3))
 (segment (start 122.431 51.611) (end 122.72 51.9) (width 0.2) (layer "F.Cu") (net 3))
 (segment (start 122.56 51.9) (end 122.72 51.9) (width 0.2) (layer "F.Cu") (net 3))
 (segment (start 104.1 50.16) (end 104.04 50.16) (width 0.2) (layer "F.Cu") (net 3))
 (via (at 122.72 51.9) (size 0.9) (drill 0.6) (layers "F.Cu" "B.Cu") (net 3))
 (segment (start 122.8 62.39) (end 122.11 63.08) (width 0.2) (layer "B.Cu") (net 3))
 (segment (start 122.11 63.08) (end 120.02 63.08) (width 0.2) (layer "B.Cu") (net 3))
 (segment (start 122.72 51.9) (end 122.72 62.31) (width 0.2) (layer "B.Cu") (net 3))
 (segment (start 122.72 62.31) (end 122.8 62.39) (width 0.2) (layer "B.Cu") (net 3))
 (segment (start 149.84 55.115) (end 152.685 52.27) (width 1) (layer "B.Cu") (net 5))
 (segment (start 154.38 60.2) (end 156.34 62.16) (width 1) (layer "B.Cu") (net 5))
 (segment (start 156.2 52.27) (end 156.32 52.39) (width 1) (layer "B.Cu") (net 5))
 (segment (start 149.84 55.115) (end 154.38 59.655) (width 1) (layer "B.Cu") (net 5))
 (segment (start 152.685 52.27) (end 156.2 52.27) (width 1) (layer "B.Cu") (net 5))
 (segment (start 154.38 59.655) (end 154.38 60.2) (width 1) (layer "B.Cu") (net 5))
 (segment (start 123.829 51.149) (end 124.34 51.66) (width 0.2) (layer "F.Cu") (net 6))
 (segment (start 112.11 49.13) (end 114.129 51.149) (width 0.2) (layer "F.Cu") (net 6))
 (segment (start 124.34 51.66) (end 124.34 52.06) (width 0.2) (layer "F.Cu") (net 6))
 (segment (start 114.129 51.149) (end 123.829 51.149) (width 0.2) (layer "F.Cu") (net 6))
 (via (at 124.34 52.06) (size 0.9) (drill 0.6) (layers "F.Cu" "B.Cu") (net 6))
 (segment (start 124.34 52.06) (end 124.49 52.06) (width 0.2) (layer "B.Cu") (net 6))
 (segment (start 124.74 58.12) (end 126.59 58.12) (width 0.2) (layer "B.Cu") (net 6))
 (segment (start 126.59 58.12) (end 126.94 57.77) (width 0.2) (layer "B.Cu") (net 6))
 (segment (start 124.34 52.21) (end 124.74 52.61) (width 0.2) (layer "B.Cu") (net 6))
 (segment (start 124.34 52.06) (end 124.34 52.21) (width 0.2) (layer "B.Cu") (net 6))
 (segment (start 124.74 52.61) (end 124.74 58.12) (width 0.2) (layer "B.Cu") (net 6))
 (segment (start 129.49 51.75) (end 126.76 51.75) (width 0.2) (layer "F.Cu") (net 7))
 (segment (start 124.81514 51.33) (end 124.10514 50.62) (width 0.2) (layer "F.Cu") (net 7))
 (segment (start 126.34 51.33) (end 124.81514 51.33) (width 0.2) (layer "F.Cu") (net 7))
 (segment (start 126.76 51.75) (end 126.34 51.33) (width 0.2) (layer "F.Cu") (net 7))
 (segment (start 129.68 51.94) (end 129.49 51.75) (width 0.2) (layer "F.Cu") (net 7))
 (segment (start 124.10514 50.62) (end 116.139999 50.62) (width 0.2) (layer "F.Cu") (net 7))
 (segment (start 116.139999 50.62) (end 114.649999 49.13) (width 0.2) (layer "F.Cu") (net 7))
 (via (at 129.68 51.94) (size 0.9) (drill 0.6) (layers "F.Cu" "B.Cu") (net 7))
 (segment (start 129.68 51.94) (end 129.95 52.21) (width 0.2) (layer "B.Cu") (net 7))
 (segment (start 129.54 60.66) (end 126.94 60.66) (width 0.2) (layer "B.Cu") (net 7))
 (segment (start 129.95 60.25) (end 129.54 60.66) (width 0.2) (layer "B.Cu") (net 7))
 (segment (start 129.95 52.21) (end 129.95 60.25) (width 0.2) (layer "B.Cu") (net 7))
 (segment (start 128.42 61.72) (end 126.94 63.2) (width 0.5) (layer "B.Cu") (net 8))
 (segment (start 131.06 61.72) (end 128.42 61.72) (width 0.5) (layer "B.Cu") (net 8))
 (segment (start 131.06 50.3) (end 131.06 61.72) (width 0.5) (layer "B.Cu") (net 8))
 (segment (start 129.89 49.13) (end 131.06 50.3) (width 0.5) (layer "B.Cu") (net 8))
 (segment (start 101.61 46.92) (end 101.560001 46.969999) (width 0.5) (layer "F.Cu") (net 2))
 (segment (start 101.560001 46.969999) (end 101.560001 50.16) (width 0.5) (layer "F.Cu") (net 2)))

